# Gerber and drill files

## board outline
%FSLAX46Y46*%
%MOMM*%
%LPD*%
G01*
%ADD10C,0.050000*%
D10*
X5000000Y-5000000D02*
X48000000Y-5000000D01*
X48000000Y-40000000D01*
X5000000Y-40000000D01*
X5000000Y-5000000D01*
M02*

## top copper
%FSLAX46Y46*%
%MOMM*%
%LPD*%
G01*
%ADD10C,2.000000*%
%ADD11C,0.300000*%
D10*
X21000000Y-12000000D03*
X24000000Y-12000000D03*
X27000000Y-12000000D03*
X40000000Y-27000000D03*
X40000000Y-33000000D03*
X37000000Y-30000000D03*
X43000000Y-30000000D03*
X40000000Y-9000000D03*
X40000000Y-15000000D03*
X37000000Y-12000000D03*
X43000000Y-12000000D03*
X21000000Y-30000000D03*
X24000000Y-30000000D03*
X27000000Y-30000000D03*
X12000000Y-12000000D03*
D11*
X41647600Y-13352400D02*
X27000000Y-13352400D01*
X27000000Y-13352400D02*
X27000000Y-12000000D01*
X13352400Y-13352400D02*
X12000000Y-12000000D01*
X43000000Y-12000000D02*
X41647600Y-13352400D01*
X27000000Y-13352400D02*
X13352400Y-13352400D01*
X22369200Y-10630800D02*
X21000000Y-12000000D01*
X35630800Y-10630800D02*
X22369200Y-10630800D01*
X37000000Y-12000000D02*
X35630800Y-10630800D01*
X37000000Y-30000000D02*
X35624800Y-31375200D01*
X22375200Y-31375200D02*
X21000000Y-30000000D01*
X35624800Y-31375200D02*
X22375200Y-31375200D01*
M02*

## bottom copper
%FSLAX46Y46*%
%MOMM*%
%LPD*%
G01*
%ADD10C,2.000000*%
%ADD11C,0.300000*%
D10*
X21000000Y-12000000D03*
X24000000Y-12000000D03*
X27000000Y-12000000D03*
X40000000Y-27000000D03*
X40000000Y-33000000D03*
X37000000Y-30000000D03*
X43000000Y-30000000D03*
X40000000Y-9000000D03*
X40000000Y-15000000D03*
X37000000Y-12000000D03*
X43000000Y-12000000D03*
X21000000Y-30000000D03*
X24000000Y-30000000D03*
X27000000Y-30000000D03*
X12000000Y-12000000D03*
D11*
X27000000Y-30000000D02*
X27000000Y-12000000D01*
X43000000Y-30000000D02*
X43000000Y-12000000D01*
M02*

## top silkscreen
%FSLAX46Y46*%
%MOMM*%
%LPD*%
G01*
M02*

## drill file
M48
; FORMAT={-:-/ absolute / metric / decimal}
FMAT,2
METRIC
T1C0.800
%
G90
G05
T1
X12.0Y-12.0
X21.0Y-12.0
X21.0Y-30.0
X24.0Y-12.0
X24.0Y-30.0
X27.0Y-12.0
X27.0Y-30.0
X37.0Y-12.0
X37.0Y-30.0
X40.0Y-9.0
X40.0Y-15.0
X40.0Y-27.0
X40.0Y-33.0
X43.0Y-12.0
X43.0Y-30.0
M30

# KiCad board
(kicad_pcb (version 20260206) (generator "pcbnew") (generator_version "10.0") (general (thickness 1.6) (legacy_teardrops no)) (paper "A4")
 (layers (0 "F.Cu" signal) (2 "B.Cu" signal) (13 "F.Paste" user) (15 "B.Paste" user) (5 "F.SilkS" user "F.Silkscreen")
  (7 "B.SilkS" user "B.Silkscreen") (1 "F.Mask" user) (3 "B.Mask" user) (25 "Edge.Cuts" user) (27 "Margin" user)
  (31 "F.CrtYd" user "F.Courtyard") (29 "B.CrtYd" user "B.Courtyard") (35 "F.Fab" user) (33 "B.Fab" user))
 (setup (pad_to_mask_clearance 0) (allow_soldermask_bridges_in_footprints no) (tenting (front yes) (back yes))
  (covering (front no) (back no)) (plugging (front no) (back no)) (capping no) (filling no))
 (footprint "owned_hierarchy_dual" (layer "F.Cu") (at 24 12)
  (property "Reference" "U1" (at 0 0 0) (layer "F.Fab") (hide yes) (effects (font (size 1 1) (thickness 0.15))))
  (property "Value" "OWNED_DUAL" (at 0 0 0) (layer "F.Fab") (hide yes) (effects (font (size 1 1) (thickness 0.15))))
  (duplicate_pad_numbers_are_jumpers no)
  (pad "1" thru_hole circle (at -3 0) (size 2 2) (drill 0.8) (layers "*.Cu" "*.Mask") (remove_unused_layers no) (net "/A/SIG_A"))
  (pad "2" thru_hole circle (at 0 0) (size 2 2) (drill 0.8) (layers "*.Cu" "*.Mask") (remove_unused_layers no) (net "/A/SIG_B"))
  (pad "3" thru_hole circle (at 3 0) (size 2 2) (drill 0.8) (layers "*.Cu" "*.Mask") (remove_unused_layers no) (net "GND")))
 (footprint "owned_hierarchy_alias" (layer "F.Cu") (at 40 30)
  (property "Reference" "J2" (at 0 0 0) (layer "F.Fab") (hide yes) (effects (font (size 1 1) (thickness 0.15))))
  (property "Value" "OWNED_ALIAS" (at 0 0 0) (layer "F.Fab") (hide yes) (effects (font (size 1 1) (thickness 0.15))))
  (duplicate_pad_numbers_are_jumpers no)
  (pad "MP" thru_hole circle (at 0 -3) (size 2 2) (drill 0.8) (layers "*.Cu" "*.Mask") (remove_unused_layers no))
  (pad "MP" thru_hole circle (at 0 3) (size 2 2) (drill 0.8) (layers "*.Cu" "*.Mask") (remove_unused_layers no))
  (pad "R" thru_hole circle (at -3 0) (size 2 2) (drill 0.8) (layers "*.Cu" "*.Mask") (remove_unused_layers no) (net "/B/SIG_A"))
  (pad "T" thru_hole circle (at 3 0) (size 2 2) (drill 0.8) (layers "*.Cu" "*.Mask") (remove_unused_layers no) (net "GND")))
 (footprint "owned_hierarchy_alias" (layer "F.Cu") (at 40 12)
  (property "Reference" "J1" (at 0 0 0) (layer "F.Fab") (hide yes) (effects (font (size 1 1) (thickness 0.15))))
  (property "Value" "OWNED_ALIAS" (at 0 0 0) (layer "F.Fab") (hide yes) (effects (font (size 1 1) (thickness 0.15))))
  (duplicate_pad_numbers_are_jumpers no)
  (pad "MP" thru_hole circle (at 0 -3) (size 2 2) (drill 0.8) (layers "*.Cu" "*.Mask") (remove_unused_layers no))
  (pad "MP" thru_hole circle (at 0 3) (size 2 2) (drill 0.8) (layers "*.Cu" "*.Mask") (remove_unused_layers no))
  (pad "R" thru_hole circle (at -3 0) (size 2 2) (drill 0.8) (layers "*.Cu" "*.Mask") (remove_unused_layers no) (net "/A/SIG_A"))
  (pad "T" thru_hole circle (at 3 0) (size 2 2) (drill 0.8) (layers "*.Cu" "*.Mask") (remove_unused_layers no) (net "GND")))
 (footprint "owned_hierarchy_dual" (layer "F.Cu") (at 24 30)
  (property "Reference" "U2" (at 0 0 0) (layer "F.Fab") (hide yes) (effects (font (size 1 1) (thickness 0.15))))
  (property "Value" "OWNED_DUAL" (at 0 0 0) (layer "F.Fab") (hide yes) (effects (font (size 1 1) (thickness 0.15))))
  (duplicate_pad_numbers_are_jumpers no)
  (pad "1" thru_hole circle (at -3 0) (size 2 2) (drill 0.8) (layers "*.Cu" "*.Mask") (remove_unused_layers no) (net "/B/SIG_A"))
  (pad "2" thru_hole circle (at 0 0) (size 2 2) (drill 0.8) (layers "*.Cu" "*.Mask") (remove_unused_layers no) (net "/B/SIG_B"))
  (pad "3" thru_hole circle (at 3 0) (size 2 2) (drill 0.8) (layers "*.Cu" "*.Mask") (remove_unused_layers no) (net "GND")))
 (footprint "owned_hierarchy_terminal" (layer "F.Cu") (at 12 12)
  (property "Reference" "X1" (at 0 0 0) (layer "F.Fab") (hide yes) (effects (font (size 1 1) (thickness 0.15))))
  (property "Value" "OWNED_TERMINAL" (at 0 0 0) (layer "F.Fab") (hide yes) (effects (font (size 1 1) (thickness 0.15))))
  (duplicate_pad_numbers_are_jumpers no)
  (pad "1" thru_hole circle (at 0 0) (size 2 2) (drill 0.8) (layers "*.Cu" "*.Mask") (remove_unused_layers no) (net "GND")))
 (gr_rect (start 5 5) (end 48 40) (stroke (width 0.05) (type default)) (fill no) (layer "Edge.Cuts"))
 (segment (start 41.6476 13.3524) (end 27 13.3524) (width 0.3) (layer "F.Cu") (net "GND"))
 (segment (start 27 13.3524) (end 27 12) (width 0.3) (layer "F.Cu") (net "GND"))
 (segment (start 13.3524 13.3524) (end 12 12) (width 0.3) (layer "F.Cu") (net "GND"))
 (segment (start 43 12) (end 41.6476 13.3524) (width 0.3) (layer "F.Cu") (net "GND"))
 (segment (start 27 13.3524) (end 13.3524 13.3524) (width 0.3) (layer "F.Cu") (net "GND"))
 (segment (start 27 30) (end 27 12) (width 0.3) (layer "B.Cu") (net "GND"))
 (segment (start 43 30) (end 43 12) (width 0.3) (layer "B.Cu") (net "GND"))
 (segment (start 22.3692 10.6308) (end 21 12) (width 0.3) (layer "F.Cu") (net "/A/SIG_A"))
 (segment (start 35.6308 10.6308) (end 22.3692 10.6308) (width 0.3) (layer "F.Cu") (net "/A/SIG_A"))
 (segment (start 37 12) (end 35.6308 10.6308) (width 0.3) (layer "F.Cu") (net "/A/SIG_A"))
 (segment (start 37 30) (end 35.6248 31.3752) (width 0.3) (layer "F.Cu") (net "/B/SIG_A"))
 (segment (start 22.3752 31.3752) (end 21 30) (width 0.3) (layer "F.Cu") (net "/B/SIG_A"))
 (segment (start 35.6248 31.3752) (end 22.3752 31.3752) (width 0.3) (layer "F.Cu") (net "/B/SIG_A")))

